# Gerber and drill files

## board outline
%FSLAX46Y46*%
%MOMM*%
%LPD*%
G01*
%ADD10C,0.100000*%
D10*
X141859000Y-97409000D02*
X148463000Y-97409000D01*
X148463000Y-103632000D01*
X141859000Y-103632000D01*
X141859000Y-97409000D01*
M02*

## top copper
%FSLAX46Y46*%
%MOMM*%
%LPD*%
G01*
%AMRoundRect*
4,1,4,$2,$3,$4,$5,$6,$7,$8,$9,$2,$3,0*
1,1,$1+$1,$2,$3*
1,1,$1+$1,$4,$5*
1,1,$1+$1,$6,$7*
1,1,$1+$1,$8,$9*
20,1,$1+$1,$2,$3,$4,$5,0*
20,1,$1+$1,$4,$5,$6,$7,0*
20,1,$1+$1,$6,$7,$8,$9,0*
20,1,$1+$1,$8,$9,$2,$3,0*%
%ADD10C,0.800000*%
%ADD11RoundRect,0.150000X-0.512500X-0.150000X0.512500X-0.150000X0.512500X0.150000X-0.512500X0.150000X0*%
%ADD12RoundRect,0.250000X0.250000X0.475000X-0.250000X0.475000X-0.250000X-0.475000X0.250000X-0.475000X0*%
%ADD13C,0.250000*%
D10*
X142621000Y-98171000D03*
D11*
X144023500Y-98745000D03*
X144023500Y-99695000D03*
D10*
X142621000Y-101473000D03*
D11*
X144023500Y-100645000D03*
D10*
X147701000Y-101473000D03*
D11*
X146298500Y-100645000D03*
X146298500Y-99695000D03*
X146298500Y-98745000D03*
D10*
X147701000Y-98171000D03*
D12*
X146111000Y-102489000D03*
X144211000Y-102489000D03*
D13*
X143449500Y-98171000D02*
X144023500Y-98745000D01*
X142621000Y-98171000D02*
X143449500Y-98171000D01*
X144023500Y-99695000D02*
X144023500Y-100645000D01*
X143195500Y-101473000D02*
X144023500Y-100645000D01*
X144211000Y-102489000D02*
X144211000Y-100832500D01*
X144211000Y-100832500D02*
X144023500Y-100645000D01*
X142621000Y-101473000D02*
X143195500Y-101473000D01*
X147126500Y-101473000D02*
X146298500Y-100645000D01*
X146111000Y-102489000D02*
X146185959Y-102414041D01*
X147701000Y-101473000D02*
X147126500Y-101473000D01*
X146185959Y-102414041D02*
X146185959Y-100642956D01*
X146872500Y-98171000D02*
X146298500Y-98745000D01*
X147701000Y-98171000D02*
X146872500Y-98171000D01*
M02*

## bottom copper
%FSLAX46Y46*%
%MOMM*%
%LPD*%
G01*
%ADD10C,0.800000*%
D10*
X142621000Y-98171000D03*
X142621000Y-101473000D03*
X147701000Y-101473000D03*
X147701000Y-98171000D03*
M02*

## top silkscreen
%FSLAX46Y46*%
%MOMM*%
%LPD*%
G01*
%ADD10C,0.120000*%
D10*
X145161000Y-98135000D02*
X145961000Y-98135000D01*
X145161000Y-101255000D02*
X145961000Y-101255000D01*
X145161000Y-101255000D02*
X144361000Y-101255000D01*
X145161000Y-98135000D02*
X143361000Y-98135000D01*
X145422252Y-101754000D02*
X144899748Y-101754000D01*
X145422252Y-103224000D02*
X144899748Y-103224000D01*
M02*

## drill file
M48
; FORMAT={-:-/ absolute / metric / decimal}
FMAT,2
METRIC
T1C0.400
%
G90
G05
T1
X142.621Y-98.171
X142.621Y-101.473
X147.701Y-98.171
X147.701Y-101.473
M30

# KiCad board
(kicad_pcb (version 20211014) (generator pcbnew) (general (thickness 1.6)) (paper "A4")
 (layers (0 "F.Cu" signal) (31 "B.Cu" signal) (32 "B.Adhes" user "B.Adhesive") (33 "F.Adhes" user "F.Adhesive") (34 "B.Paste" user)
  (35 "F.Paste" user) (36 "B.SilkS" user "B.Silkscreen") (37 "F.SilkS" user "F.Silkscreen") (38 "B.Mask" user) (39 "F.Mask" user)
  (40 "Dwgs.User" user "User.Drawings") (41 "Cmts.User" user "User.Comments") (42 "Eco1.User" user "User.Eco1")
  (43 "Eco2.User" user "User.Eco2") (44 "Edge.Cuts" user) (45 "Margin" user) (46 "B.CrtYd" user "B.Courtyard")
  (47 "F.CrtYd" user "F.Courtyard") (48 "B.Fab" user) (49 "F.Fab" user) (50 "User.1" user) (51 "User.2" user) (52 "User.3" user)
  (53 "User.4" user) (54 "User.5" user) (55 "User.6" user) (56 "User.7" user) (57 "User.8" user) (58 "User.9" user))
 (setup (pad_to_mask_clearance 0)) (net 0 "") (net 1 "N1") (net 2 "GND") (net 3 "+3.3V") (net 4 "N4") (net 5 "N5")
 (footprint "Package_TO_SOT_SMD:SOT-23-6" (layer "F.Cu") (at 145.161 99.695)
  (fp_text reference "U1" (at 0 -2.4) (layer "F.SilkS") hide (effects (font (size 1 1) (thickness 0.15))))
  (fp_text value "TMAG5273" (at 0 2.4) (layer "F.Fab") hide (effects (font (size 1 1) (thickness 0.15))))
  (fp_line (start 0 -1.56) (end 0.8 -1.56) (layer "F.SilkS") (width 0.12))
  (fp_line (start 0 1.56) (end 0.8 1.56) (layer "F.SilkS") (width 0.12))
  (fp_line (start 0 1.56) (end -0.8 1.56) (layer "F.SilkS") (width 0.12))
  (fp_line (start 0 -1.56) (end -1.8 -1.56) (layer "F.SilkS") (width 0.12))
  (pad "1" thru_hole circle (at -2.54 -1.524) (size 0.8 0.8) (drill 0.4) (layers *.Cu *.Mask) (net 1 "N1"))
  (pad "1" smd roundrect (at -1.1375 -0.95) (size 1.325 0.6) (layers "F.Cu" "F.Paste" "F.Mask") (roundrect_rratio 0.25) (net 1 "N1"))
  (pad "2" smd roundrect (at -1.1375 0) (size 1.325 0.6) (layers "F.Cu" "F.Paste" "F.Mask") (roundrect_rratio 0.25) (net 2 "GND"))
  (pad "3" thru_hole circle (at -2.54 1.778) (size 0.8 0.8) (drill 0.4) (layers *.Cu *.Mask) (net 2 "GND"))
  (pad "3" smd roundrect (at -1.1375 0.95) (size 1.325 0.6) (layers "F.Cu" "F.Paste" "F.Mask") (roundrect_rratio 0.25) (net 2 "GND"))
  (pad "4" thru_hole circle (at 2.54 1.778) (size 0.8 0.8) (drill 0.4) (layers *.Cu *.Mask) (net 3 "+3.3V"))
  (pad "4" smd roundrect (at 1.1375 0.95) (size 1.325 0.6) (layers "F.Cu" "F.Paste" "F.Mask") (roundrect_rratio 0.25) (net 3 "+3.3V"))
  (pad "5" smd roundrect (at 1.1375 0) (size 1.325 0.6) (layers "F.Cu" "F.Paste" "F.Mask") (roundrect_rratio 0.25) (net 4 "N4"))
  (pad "6" smd roundrect (at 1.1375 -0.95) (size 1.325 0.6) (layers "F.Cu" "F.Paste" "F.Mask") (roundrect_rratio 0.25) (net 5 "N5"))
  (pad "6" thru_hole circle (at 2.54 -1.524) (size 0.8 0.8) (drill 0.4) (layers *.Cu *.Mask) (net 5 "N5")))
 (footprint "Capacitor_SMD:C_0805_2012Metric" (layer "F.Cu") (at 145.161 102.489 180)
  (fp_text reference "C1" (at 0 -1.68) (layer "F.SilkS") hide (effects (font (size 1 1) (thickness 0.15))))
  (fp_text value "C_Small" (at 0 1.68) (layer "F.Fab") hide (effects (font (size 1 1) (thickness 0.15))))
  (fp_line (start -0.261252 0.735) (end 0.261252 0.735) (layer "F.SilkS") (width 0.12))
  (fp_line (start -0.261252 -0.735) (end 0.261252 -0.735) (layer "F.SilkS") (width 0.12))
  (pad "1" smd roundrect (at -0.95 0 180) (size 1 1.45) (layers "F.Cu" "F.Paste" "F.Mask") (roundrect_rratio 0.25) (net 3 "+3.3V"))
  (pad "2" smd roundrect (at 0.95 0 180) (size 1 1.45) (layers "F.Cu" "F.Paste" "F.Mask") (roundrect_rratio 0.25) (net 2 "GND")))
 (gr_rect (start 141.859 97.409) (end 148.463 103.632) (layer "Edge.Cuts") (width 0.1) (fill none))
 (segment (start 143.4495 98.171) (end 144.0235 98.745) (width 0.25) (layer "F.Cu") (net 1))
 (segment (start 142.621 98.171) (end 143.4495 98.171) (width 0.25) (layer "F.Cu") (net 1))
 (segment (start 144.0235 99.695) (end 144.0235 100.645) (width 0.25) (layer "F.Cu") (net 2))
 (segment (start 143.1955 101.473) (end 144.0235 100.645) (width 0.25) (layer "F.Cu") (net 2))
 (segment (start 144.211 102.489) (end 144.211 100.8325) (width 0.25) (layer "F.Cu") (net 2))
 (segment (start 144.211 100.8325) (end 144.0235 100.645) (width 0.25) (layer "F.Cu") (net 2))
 (segment (start 142.621 101.473) (end 143.1955 101.473) (width 0.25) (layer "F.Cu") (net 2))
 (segment (start 147.1265 101.473) (end 146.2985 100.645) (width 0.25) (layer "F.Cu") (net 3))
 (segment (start 146.111 102.489) (end 146.185959 102.414041) (width 0.25) (layer "F.Cu") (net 3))
 (segment (start 147.701 101.473) (end 147.1265 101.473) (width 0.25) (layer "F.Cu") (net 3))
 (segment (start 146.185959 102.414041) (end 146.185959 100.642956) (width 0.25) (layer "F.Cu") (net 3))
 (segment (start 146.8725 98.171) (end 146.2985 98.745) (width 0.25) (layer "F.Cu") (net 5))
 (segment (start 147.701 98.171) (end 146.8725 98.171) (width 0.25) (layer "F.Cu") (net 5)))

